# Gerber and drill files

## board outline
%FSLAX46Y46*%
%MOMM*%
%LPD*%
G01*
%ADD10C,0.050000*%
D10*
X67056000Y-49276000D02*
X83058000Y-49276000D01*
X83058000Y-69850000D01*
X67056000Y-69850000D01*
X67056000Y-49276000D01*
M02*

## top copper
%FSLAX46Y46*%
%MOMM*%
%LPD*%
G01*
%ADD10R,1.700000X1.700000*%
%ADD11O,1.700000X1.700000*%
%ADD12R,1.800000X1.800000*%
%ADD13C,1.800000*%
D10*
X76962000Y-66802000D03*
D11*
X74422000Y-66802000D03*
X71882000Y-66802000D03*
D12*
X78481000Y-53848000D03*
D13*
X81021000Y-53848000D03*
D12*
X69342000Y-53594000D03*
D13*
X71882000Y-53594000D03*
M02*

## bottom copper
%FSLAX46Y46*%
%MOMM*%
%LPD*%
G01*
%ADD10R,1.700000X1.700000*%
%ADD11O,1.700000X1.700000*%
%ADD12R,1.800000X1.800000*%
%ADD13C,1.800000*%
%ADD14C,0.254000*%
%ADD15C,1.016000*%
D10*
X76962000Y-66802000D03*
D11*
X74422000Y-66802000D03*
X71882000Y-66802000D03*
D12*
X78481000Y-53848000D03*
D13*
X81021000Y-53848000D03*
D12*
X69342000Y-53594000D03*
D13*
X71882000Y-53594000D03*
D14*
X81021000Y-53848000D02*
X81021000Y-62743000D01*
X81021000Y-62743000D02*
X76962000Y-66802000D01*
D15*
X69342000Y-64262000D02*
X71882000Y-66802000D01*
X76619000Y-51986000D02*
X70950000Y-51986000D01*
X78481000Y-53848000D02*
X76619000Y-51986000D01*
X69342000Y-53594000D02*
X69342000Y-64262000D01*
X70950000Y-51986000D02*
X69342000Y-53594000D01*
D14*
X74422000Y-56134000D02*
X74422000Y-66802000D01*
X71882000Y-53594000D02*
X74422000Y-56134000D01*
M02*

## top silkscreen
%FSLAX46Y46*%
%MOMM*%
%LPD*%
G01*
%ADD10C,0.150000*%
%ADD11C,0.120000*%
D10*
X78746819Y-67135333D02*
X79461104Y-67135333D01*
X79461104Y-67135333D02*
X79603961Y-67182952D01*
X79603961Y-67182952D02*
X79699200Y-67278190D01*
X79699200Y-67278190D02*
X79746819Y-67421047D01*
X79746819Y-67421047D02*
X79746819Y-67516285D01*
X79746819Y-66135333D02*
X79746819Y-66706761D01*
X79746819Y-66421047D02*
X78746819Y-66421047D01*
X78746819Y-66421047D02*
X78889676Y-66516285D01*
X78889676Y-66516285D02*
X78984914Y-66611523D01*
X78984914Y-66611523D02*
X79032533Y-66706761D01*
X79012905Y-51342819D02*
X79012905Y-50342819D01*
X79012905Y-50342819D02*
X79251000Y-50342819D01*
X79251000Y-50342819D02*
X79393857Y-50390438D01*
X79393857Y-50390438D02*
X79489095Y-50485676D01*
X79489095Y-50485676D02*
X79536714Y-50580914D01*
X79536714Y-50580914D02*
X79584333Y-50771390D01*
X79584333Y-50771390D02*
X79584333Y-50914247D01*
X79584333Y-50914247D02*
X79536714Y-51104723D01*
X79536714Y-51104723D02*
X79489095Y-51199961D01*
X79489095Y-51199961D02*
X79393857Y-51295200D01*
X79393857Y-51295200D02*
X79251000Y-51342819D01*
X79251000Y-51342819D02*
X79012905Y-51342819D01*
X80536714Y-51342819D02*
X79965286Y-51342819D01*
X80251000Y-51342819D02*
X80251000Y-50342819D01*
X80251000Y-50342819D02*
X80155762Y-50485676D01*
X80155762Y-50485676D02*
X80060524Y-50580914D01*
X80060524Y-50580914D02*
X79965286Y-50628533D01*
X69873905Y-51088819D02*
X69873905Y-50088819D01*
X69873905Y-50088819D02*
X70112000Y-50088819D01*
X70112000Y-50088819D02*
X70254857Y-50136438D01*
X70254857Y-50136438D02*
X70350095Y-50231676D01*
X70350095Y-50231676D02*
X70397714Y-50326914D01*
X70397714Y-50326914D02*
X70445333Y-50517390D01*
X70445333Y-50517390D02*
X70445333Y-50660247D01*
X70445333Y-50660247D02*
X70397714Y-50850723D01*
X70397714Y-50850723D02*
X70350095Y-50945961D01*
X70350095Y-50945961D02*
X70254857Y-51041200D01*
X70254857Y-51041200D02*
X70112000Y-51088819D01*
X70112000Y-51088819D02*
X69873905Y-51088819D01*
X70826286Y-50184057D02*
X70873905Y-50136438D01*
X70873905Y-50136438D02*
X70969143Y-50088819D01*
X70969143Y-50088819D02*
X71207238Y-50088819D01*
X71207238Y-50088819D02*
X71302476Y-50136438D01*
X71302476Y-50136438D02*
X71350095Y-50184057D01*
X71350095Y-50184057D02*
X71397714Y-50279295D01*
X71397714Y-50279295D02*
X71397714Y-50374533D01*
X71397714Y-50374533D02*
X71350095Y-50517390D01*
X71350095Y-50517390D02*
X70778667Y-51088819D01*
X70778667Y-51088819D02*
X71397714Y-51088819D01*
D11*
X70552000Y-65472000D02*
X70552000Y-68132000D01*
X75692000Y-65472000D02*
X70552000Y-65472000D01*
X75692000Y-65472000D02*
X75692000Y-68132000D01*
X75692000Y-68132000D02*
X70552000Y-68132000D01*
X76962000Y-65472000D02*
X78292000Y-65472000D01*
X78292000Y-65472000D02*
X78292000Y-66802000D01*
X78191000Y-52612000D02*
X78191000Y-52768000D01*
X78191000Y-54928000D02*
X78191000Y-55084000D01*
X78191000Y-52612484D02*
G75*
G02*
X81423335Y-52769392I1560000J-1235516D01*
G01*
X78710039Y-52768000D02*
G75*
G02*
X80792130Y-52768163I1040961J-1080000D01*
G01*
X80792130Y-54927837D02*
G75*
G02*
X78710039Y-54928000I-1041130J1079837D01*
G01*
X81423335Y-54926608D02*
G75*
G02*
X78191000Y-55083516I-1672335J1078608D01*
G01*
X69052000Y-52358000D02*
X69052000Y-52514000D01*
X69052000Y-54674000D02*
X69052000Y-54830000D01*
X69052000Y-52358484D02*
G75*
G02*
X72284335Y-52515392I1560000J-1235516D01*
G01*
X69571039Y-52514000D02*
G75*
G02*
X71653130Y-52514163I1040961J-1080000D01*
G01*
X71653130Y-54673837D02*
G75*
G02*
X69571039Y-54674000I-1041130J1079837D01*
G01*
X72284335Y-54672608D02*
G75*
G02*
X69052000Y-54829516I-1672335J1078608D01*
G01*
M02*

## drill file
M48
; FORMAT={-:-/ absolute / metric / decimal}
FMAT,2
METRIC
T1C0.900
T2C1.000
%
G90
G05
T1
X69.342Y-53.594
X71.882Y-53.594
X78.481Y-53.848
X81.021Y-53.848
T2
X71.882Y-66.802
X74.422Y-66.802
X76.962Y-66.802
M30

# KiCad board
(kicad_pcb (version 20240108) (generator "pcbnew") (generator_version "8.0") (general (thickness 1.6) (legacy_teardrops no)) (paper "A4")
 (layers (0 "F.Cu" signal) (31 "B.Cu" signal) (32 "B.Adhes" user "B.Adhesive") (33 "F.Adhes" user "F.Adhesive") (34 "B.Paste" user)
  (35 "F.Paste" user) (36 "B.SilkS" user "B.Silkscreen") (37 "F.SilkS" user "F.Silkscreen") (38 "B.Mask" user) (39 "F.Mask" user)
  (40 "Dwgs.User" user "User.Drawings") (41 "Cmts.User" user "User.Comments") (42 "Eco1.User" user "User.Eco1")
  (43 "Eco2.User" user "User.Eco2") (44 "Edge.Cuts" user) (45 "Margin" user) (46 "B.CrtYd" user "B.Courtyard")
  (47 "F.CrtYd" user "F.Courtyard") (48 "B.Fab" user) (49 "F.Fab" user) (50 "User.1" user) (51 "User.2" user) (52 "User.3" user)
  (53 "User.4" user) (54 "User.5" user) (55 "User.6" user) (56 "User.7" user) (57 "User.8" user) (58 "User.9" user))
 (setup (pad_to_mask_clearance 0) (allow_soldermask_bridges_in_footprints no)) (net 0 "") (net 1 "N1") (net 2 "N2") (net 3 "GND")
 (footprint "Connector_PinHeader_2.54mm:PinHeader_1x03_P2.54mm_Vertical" (layer "F.Cu") (at 76.962 66.802 -90)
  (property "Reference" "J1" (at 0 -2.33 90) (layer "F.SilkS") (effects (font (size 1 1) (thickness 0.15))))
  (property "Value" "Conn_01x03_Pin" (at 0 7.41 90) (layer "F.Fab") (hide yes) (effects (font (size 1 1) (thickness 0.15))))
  (fp_line (start -1.33 6.41) (end 1.33 6.41) (stroke (width 0.12) (type solid)) (layer "F.SilkS"))
  (fp_line (start -1.33 1.27) (end -1.33 6.41) (stroke (width 0.12) (type solid)) (layer "F.SilkS"))
  (fp_line (start -1.33 1.27) (end 1.33 1.27) (stroke (width 0.12) (type solid)) (layer "F.SilkS"))
  (fp_line (start 1.33 1.27) (end 1.33 6.41) (stroke (width 0.12) (type solid)) (layer "F.SilkS"))
  (fp_line (start -1.33 0) (end -1.33 -1.33) (stroke (width 0.12) (type solid)) (layer "F.SilkS"))
  (fp_line (start -1.33 -1.33) (end 0 -1.33) (stroke (width 0.12) (type solid)) (layer "F.SilkS"))
  (pad "1" thru_hole rect (at 0 0 270) (size 1.7 1.7) (drill 1) (layers "*.Cu" "*.Mask") (remove_unused_layers no) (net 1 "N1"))
  (pad "2" thru_hole oval (at 0 2.54 270) (size 1.7 1.7) (drill 1) (layers "*.Cu" "*.Mask") (remove_unused_layers no) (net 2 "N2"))
  (pad "3" thru_hole oval (at 0 5.08 270) (size 1.7 1.7) (drill 1) (layers "*.Cu" "*.Mask") (remove_unused_layers no) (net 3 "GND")))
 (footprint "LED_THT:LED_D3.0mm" (layer "F.Cu") (at 78.481 53.848)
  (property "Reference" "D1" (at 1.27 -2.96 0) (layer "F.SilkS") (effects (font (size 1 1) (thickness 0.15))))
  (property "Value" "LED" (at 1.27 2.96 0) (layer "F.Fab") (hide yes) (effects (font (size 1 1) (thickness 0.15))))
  (fp_line (start -0.29 -1.236) (end -0.29 -1.08) (stroke (width 0.12) (type solid)) (layer "F.SilkS"))
  (fp_line (start -0.29 1.08) (end -0.29 1.236) (stroke (width 0.12) (type solid)) (layer "F.SilkS"))
  (fp_arc (start -0.29 -1.235516) (mid 1.366487 -1.987659) (end 2.942335 -1.078608) (stroke (width 0.12) (type solid)) (layer "F.SilkS"))
  (fp_arc (start 0.229039 -1.08) (mid 1.270117 -1.5) (end 2.31113 -1.079837) (stroke (width 0.12) (type solid)) (layer "F.SilkS"))
  (fp_arc (start 2.31113 1.079837) (mid 1.270117 1.5) (end 0.229039 1.08) (stroke (width 0.12) (type solid)) (layer "F.SilkS"))
  (fp_arc (start 2.942335 1.078608) (mid 1.366487 1.987659) (end -0.29 1.235516) (stroke (width 0.12) (type solid)) (layer "F.SilkS"))
  (pad "1" thru_hole rect (at 0 0) (size 1.8 1.8) (drill 0.9) (layers "*.Cu" "*.Mask") (remove_unused_layers no) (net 3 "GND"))
  (pad "2" thru_hole circle (at 2.54 0) (size 1.8 1.8) (drill 0.9) (layers "*.Cu" "*.Mask") (remove_unused_layers no) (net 1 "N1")))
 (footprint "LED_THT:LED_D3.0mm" (layer "F.Cu") (at 69.342 53.594)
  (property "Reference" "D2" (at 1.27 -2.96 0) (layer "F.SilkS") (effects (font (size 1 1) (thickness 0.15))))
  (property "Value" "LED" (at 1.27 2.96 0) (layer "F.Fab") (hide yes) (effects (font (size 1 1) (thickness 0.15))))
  (fp_line (start -0.29 -1.236) (end -0.29 -1.08) (stroke (width 0.12) (type solid)) (layer "F.SilkS"))
  (fp_line (start -0.29 1.08) (end -0.29 1.236) (stroke (width 0.12) (type solid)) (layer "F.SilkS"))
  (fp_arc (start -0.29 -1.235516) (mid 1.366487 -1.987659) (end 2.942335 -1.078608) (stroke (width 0.12) (type solid)) (layer "F.SilkS"))
  (fp_arc (start 0.229039 -1.08) (mid 1.270117 -1.5) (end 2.31113 -1.079837) (stroke (width 0.12) (type solid)) (layer "F.SilkS"))
  (fp_arc (start 2.31113 1.079837) (mid 1.270117 1.5) (end 0.229039 1.08) (stroke (width 0.12) (type solid)) (layer "F.SilkS"))
  (fp_arc (start 2.942335 1.078608) (mid 1.366487 1.987659) (end -0.29 1.235516) (stroke (width 0.12) (type solid)) (layer "F.SilkS"))
  (pad "1" thru_hole rect (at 0 0) (size 1.8 1.8) (drill 0.9) (layers "*.Cu" "*.Mask") (remove_unused_layers no) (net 3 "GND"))
  (pad "2" thru_hole circle (at 2.54 0) (size 1.8 1.8) (drill 0.9) (layers "*.Cu" "*.Mask") (remove_unused_layers no) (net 2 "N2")))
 (gr_rect (start 67.056 49.276) (end 83.058 69.85) (stroke (width 0.05) (type default)) (fill none) (layer "Edge.Cuts"))
 (segment (start 81.021 53.848) (end 81.021 62.743) (width 0.254) (layer "B.Cu") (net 1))
 (segment (start 81.021 62.743) (end 76.962 66.802) (width 0.254) (layer "B.Cu") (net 1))
 (segment (start 69.342 64.262) (end 71.882 66.802) (width 1.016) (layer "B.Cu") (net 3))
 (segment (start 76.619 51.986) (end 70.95 51.986) (width 1.016) (layer "B.Cu") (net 3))
 (segment (start 78.481 53.848) (end 76.619 51.986) (width 1.016) (layer "B.Cu") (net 3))
 (segment (start 69.342 53.594) (end 69.342 64.262) (width 1.016) (layer "B.Cu") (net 3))
 (segment (start 70.95 51.986) (end 69.342 53.594) (width 1.016) (layer "B.Cu") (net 3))
 (segment (start 74.422 56.134) (end 74.422 66.802) (width 0.254) (layer "B.Cu") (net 2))
 (segment (start 71.882 53.594) (end 74.422 56.134) (width 0.254) (layer "B.Cu") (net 2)))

